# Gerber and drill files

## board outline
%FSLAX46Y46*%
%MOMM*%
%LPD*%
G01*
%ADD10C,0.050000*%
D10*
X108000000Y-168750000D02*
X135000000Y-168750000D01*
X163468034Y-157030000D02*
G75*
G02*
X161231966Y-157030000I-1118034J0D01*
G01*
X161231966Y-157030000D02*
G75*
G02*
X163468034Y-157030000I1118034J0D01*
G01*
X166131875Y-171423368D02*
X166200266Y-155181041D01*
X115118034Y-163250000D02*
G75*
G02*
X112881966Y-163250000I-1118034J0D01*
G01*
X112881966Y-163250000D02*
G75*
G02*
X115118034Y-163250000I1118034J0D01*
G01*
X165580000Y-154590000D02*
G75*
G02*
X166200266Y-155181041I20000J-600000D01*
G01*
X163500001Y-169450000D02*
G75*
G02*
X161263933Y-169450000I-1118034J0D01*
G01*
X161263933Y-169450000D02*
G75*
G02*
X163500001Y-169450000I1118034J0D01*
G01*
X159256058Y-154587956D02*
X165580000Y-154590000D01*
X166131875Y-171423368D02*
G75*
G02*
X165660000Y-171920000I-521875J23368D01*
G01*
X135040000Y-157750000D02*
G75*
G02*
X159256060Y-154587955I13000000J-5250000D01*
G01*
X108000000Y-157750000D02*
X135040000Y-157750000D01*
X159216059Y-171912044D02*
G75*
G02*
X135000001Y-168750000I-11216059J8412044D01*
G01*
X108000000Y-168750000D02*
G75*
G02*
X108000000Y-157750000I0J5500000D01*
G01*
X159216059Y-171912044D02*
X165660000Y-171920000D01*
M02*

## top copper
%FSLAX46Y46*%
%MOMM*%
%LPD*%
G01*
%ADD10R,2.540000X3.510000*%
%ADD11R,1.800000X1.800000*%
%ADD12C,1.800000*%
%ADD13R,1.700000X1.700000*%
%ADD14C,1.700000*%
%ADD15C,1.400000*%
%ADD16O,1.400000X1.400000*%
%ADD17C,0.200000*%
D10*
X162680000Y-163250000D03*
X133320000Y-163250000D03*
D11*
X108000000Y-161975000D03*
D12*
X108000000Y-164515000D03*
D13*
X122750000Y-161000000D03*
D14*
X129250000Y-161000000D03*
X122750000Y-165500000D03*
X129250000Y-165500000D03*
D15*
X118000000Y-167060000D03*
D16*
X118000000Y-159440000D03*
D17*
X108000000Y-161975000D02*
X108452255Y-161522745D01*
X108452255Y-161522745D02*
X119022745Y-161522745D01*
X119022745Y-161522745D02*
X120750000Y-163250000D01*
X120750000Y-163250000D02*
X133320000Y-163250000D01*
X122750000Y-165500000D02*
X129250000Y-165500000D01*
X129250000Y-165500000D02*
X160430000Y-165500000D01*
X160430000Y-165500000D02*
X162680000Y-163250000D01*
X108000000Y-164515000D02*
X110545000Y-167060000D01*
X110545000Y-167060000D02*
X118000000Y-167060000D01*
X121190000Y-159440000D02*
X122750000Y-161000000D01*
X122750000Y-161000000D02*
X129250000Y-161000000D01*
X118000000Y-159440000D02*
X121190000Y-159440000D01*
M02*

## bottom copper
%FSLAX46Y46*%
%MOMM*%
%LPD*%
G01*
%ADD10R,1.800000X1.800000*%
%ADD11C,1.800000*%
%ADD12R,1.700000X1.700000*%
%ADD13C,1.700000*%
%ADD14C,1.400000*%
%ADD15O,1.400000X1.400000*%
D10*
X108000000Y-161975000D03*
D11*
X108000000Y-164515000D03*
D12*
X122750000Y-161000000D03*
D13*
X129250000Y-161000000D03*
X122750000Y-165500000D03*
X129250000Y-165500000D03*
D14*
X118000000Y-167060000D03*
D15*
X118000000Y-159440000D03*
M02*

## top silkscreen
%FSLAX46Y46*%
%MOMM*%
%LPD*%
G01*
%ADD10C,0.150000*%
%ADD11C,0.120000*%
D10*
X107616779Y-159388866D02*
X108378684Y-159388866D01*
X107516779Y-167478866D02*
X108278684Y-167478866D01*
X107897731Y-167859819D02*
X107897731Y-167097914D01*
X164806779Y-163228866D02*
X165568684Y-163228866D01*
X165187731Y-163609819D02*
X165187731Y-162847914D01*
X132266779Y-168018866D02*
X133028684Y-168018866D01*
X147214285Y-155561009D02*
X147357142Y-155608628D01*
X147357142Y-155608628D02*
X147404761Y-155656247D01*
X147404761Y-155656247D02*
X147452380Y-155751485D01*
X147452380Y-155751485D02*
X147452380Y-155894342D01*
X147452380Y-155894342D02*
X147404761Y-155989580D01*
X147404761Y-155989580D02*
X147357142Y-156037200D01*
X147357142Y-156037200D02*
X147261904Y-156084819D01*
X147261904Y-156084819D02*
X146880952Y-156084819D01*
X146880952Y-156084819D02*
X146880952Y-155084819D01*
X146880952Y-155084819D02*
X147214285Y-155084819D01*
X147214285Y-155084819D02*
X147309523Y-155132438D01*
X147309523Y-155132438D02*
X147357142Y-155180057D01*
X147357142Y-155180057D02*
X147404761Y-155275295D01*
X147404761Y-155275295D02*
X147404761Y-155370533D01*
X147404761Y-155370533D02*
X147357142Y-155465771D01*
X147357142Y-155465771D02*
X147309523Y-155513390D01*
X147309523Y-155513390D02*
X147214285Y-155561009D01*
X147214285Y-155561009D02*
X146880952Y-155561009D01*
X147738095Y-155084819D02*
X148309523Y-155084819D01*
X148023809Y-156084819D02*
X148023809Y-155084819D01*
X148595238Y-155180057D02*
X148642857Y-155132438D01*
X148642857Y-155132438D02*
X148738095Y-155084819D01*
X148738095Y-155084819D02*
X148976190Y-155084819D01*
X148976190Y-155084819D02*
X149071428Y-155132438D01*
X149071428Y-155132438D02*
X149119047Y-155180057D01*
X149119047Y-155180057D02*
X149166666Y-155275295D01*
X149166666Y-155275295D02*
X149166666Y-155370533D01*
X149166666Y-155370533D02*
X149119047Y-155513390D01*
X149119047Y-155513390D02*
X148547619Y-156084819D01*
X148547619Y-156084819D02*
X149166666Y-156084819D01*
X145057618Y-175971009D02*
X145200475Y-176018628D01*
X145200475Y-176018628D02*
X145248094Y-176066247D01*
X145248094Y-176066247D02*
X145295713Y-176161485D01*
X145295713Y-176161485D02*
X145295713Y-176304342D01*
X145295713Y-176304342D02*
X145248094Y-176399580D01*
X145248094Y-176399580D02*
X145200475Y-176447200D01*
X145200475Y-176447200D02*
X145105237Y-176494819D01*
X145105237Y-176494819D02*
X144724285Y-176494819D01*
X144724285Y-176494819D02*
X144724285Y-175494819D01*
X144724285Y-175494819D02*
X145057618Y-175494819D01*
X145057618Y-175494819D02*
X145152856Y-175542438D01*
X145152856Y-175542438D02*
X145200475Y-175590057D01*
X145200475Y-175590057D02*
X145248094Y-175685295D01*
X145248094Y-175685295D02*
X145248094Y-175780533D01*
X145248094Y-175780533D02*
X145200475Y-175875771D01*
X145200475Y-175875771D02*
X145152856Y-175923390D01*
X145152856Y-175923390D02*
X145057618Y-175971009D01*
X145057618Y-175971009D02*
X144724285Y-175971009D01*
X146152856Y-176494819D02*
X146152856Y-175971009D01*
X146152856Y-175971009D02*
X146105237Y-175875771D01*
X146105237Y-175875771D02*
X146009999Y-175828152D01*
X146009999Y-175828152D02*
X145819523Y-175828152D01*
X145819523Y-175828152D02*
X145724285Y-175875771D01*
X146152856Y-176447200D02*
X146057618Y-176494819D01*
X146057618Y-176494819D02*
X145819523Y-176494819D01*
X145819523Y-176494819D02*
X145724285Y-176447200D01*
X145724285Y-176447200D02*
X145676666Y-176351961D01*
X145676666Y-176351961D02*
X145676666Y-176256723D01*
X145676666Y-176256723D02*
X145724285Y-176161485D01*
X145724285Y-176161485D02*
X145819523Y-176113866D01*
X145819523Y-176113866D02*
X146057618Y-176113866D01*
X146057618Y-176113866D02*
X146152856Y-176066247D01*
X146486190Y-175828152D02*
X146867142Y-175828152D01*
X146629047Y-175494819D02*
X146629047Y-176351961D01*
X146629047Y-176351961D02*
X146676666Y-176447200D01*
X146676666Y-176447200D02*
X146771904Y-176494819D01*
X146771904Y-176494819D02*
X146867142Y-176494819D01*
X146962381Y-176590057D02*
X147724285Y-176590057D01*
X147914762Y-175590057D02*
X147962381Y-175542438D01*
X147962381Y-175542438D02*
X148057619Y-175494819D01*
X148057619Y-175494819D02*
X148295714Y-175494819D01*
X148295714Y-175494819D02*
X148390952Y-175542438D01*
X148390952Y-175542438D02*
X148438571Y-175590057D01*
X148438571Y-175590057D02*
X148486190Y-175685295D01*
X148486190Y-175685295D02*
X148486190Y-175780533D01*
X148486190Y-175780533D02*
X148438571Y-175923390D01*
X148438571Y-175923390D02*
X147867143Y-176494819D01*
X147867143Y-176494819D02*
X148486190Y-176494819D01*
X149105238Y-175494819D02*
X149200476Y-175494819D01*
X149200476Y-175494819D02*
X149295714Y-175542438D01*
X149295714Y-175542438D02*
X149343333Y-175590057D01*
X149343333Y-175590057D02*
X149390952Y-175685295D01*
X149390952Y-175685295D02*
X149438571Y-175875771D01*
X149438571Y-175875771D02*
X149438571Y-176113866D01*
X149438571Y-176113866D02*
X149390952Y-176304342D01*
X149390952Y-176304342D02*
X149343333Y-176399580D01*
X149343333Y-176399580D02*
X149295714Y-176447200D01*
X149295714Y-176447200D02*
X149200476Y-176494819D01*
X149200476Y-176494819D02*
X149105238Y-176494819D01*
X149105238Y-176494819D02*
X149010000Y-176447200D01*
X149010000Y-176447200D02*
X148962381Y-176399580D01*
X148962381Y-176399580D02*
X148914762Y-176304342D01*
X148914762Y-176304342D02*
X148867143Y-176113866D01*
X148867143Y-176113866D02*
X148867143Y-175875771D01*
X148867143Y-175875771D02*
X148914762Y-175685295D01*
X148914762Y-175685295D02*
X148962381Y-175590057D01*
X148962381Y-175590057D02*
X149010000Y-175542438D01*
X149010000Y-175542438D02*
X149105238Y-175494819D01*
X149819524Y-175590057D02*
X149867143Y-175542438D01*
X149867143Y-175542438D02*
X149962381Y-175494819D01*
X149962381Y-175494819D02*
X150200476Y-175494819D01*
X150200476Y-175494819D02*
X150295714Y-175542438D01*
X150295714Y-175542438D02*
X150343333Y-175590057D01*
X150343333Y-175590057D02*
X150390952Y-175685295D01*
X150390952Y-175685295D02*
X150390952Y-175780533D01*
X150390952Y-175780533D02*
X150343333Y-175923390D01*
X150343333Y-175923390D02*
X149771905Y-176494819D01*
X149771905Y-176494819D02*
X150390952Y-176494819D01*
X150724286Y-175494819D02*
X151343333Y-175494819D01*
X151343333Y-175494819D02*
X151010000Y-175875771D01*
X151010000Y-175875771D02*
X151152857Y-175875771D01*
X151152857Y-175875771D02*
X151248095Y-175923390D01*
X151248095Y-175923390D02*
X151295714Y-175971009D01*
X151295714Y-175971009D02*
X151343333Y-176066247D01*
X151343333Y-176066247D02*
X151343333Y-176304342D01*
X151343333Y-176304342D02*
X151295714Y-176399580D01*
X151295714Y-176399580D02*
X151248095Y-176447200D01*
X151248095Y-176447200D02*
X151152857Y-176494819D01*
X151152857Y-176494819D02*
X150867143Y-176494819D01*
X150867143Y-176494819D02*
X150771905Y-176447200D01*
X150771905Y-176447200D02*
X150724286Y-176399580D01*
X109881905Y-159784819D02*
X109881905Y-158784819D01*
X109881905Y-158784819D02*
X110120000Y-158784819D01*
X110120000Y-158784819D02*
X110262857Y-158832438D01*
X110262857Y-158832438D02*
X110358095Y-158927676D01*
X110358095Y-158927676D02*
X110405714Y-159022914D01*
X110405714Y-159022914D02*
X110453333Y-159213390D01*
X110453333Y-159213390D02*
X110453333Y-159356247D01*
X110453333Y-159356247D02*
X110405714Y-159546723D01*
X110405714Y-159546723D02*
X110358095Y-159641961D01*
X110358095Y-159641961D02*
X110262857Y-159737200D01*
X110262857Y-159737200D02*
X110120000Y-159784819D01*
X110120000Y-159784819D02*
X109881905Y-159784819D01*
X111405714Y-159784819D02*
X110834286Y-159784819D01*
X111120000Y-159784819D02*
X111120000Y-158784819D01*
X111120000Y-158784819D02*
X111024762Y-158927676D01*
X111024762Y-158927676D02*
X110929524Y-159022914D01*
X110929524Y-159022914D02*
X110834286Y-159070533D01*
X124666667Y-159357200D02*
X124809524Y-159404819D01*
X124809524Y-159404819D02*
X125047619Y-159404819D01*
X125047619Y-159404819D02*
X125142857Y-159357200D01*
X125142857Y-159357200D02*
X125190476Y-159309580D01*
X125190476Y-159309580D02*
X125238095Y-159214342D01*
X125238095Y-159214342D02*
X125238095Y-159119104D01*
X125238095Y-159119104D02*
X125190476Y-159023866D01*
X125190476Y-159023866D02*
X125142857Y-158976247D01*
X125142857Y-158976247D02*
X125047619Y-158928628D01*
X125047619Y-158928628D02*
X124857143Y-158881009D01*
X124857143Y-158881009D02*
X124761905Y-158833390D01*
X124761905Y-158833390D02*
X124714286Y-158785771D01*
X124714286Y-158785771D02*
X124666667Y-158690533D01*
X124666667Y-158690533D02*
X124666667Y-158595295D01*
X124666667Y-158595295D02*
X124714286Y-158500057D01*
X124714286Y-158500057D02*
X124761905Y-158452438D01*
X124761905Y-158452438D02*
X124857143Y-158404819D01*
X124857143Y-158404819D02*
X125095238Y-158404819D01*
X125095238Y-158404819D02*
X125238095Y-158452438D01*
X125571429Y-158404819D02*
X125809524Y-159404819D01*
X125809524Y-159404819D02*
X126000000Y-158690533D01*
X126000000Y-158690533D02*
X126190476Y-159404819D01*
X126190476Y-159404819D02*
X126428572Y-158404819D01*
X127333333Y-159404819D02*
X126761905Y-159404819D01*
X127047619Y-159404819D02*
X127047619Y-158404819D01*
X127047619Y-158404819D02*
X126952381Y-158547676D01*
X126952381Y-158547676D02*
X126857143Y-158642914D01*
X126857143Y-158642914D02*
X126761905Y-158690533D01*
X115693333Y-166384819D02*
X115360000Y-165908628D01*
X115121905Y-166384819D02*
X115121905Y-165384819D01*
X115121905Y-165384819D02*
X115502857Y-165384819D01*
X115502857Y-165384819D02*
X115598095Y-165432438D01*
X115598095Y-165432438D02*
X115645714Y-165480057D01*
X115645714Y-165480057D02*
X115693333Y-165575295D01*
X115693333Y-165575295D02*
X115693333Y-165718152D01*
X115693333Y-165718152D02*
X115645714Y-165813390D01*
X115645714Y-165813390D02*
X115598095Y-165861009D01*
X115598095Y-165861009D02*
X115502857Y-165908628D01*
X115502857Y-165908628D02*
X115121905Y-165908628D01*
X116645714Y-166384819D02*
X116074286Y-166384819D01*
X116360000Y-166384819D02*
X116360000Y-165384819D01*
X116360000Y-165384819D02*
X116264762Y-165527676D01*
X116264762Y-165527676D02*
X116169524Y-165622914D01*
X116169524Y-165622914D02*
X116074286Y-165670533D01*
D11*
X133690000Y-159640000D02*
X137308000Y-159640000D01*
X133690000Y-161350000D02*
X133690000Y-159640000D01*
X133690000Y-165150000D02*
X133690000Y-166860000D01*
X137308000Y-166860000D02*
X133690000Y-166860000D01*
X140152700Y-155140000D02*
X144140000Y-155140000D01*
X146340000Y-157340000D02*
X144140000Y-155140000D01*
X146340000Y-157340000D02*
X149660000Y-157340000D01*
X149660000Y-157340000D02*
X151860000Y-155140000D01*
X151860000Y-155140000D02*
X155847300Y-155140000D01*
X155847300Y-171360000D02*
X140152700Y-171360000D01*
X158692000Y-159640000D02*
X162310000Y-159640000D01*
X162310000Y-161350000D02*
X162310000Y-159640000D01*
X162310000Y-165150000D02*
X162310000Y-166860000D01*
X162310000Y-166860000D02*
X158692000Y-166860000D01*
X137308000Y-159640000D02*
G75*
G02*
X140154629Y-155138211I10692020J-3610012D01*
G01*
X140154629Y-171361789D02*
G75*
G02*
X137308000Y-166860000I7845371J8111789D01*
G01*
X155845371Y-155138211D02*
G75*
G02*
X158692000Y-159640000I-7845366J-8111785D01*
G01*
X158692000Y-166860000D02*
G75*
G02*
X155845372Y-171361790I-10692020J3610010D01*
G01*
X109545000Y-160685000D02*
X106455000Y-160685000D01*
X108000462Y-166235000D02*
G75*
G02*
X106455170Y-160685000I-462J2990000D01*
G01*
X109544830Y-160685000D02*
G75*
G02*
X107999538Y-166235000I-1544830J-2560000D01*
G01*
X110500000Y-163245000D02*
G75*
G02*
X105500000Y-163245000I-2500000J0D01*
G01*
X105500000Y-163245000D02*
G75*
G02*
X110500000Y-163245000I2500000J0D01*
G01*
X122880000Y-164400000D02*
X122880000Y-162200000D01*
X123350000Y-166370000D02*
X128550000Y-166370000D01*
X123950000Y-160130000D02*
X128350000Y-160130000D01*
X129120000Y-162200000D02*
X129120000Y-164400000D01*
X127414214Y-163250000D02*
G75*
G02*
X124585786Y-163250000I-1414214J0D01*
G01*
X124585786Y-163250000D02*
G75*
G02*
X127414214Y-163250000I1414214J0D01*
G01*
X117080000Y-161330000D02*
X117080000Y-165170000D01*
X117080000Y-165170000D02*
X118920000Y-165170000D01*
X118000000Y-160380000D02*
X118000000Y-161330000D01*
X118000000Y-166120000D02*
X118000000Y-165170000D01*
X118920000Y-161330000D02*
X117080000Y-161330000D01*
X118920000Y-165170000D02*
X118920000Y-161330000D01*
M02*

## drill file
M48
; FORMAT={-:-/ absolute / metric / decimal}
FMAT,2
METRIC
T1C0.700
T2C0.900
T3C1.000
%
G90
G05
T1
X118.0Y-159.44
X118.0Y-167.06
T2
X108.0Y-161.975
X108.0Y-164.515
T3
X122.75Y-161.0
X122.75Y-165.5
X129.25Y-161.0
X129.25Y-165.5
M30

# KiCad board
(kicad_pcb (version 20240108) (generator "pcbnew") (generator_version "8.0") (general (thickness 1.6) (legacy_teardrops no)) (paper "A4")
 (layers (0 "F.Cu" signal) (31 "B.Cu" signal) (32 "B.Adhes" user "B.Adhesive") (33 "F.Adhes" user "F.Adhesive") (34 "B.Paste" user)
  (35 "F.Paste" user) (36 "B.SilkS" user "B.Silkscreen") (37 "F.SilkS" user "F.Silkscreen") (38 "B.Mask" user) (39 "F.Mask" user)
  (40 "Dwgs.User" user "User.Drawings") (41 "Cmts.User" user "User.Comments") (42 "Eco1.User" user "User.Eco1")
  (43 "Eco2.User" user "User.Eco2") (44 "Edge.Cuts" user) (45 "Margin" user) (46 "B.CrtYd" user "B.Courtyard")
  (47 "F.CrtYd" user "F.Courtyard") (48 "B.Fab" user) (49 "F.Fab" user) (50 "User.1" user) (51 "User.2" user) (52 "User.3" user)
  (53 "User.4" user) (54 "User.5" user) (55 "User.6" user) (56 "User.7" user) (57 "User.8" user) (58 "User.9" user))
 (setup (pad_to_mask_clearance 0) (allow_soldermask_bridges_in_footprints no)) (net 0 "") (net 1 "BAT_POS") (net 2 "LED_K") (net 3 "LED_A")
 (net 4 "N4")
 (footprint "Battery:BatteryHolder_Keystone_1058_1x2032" (layer "F.Cu") (at 148 163.25 180)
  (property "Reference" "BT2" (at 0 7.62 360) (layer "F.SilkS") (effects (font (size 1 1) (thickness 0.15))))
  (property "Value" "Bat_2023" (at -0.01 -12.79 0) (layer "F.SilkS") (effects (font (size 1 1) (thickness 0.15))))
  (fp_line (start 14.31 3.61) (end 10.692 3.61) (stroke (width 0.12) (type solid)) (layer "F.SilkS"))
  (fp_line (start 14.31 1.9) (end 14.31 3.61) (stroke (width 0.12) (type solid)) (layer "F.SilkS"))
  (fp_line (start 14.31 -1.9) (end 14.31 -3.61) (stroke (width 0.12) (type solid)) (layer "F.SilkS"))
  (fp_line (start 10.692 -3.61) (end 14.31 -3.61) (stroke (width 0.12) (type solid)) (layer "F.SilkS"))
  (fp_line (start 7.8473 8.11) (end 3.86 8.11) (stroke (width 0.12) (type solid)) (layer "F.SilkS"))
  (fp_line (start 1.66 5.91) (end 3.86 8.11) (stroke (width 0.12) (type solid)) (layer "F.SilkS"))
  (fp_line (start 1.66 5.91) (end -1.66 5.91) (stroke (width 0.12) (type solid)) (layer "F.SilkS"))
  (fp_line (start -1.66 5.91) (end -3.86 8.11) (stroke (width 0.12) (type solid)) (layer "F.SilkS"))
  (fp_line (start -3.86 8.11) (end -7.8473 8.11) (stroke (width 0.12) (type solid)) (layer "F.SilkS"))
  (fp_line (start -7.8473 -8.11) (end 7.8473 -8.11) (stroke (width 0.12) (type solid)) (layer "F.SilkS"))
  (fp_line (start -10.692 3.61) (end -14.31 3.61) (stroke (width 0.12) (type solid)) (layer "F.SilkS"))
  (fp_line (start -14.31 1.9) (end -14.31 3.61) (stroke (width 0.12) (type solid)) (layer "F.SilkS"))
  (fp_line (start -14.31 -1.9) (end -14.31 -3.61) (stroke (width 0.12) (type solid)) (layer "F.SilkS"))
  (fp_line (start -14.31 -3.61) (end -10.692 -3.61) (stroke (width 0.12) (type solid)) (layer "F.SilkS"))
  (fp_arc (start 10.692 3.61) (mid 9.538084 6.031244) (end 7.845371 8.111789) (stroke (width 0.12) (type solid)) (layer "F.SilkS"))
  (fp_arc (start 7.845371 -8.111789) (mid 9.538085 -6.031244) (end 10.692 -3.61) (stroke (width 0.12) (type solid)) (layer "F.SilkS"))
  (fp_arc (start -7.845371 8.111789) (mid -9.538085 6.031244) (end -10.692 3.61) (stroke (width 0.12) (type solid)) (layer "F.SilkS"))
  (fp_arc (start -10.692 -3.61) (mid -9.538084 -6.031244) (end -7.845371 -8.111789) (stroke (width 0.12) (type solid)) (layer "F.SilkS"))
  (pad "1" smd rect (at -14.68 0 180) (size 2.54 3.51) (layers "F.Cu" "F.Paste" "F.Mask") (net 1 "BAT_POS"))
  (pad "2" smd rect (at 14.68 0 180) (size 2.54 3.51) (layers "F.Cu" "F.Paste" "F.Mask") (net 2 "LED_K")))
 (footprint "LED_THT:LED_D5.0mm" (layer "F.Cu") (at 108 161.975 -90)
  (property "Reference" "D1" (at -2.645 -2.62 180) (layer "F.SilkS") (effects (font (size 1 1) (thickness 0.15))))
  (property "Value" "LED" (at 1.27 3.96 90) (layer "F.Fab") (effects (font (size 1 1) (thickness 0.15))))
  (fp_line (start -1.29 -1.545) (end -1.29 1.545) (stroke (width 0.12) (type solid)) (layer "F.SilkS"))
  (fp_arc (start 4.26 -0.000462) (mid 2.072002 2.880433) (end -1.29 1.54483) (stroke (width 0.12) (type solid)) (layer "F.SilkS"))
  (fp_arc (start -1.29 -1.54483) (mid 2.072002 -2.880433) (end 4.26 0.000462) (stroke (width 0.12) (type solid)) (layer "F.SilkS"))
  (fp_circle (center 1.27 0) (end 3.77 0) (stroke (width 0.12) (type solid)) (fill none) (layer "F.SilkS"))
  (pad "1" thru_hole rect (at 0 0 270) (size 1.8 1.8) (drill 0.9) (layers "*.Cu" "*.Mask") (remove_unused_layers no) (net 2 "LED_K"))
  (pad "2" thru_hole circle (at 2.54 0 270) (size 1.8 1.8) (drill 0.9) (layers "*.Cu" "*.Mask") (remove_unused_layers no) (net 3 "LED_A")))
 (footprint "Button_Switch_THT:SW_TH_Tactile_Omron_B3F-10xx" (layer "F.Cu") (at 122.75 161)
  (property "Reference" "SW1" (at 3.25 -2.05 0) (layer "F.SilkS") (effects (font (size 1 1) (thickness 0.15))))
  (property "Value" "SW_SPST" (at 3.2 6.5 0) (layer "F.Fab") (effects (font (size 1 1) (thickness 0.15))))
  (fp_line (start 0.13 3.4) (end 0.13 1.2) (stroke (width 0.12) (type solid)) (layer "F.SilkS"))
  (fp_line (start 0.6 5.37) (end 5.8 5.37) (stroke (width 0.12) (type solid)) (layer "F.SilkS"))
  (fp_line (start 1.2 -0.87) (end 5.6 -0.87) (stroke (width 0.12) (type solid)) (layer "F.SilkS"))
  (fp_line (start 6.37 1.2) (end 6.37 3.4) (stroke (width 0.12) (type solid)) (layer "F.SilkS"))
  (fp_circle (center 3.25 2.25) (end 4.25 3.25) (stroke (width 0.12) (type solid)) (fill none) (layer "F.SilkS"))
  (pad "1" thru_hole rect (at 0 0) (size 1.7 1.7) (drill 1) (layers "*.Cu" "*.Mask") (remove_unused_layers no) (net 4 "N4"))
  (pad "1" thru_hole circle (at 6.5 0) (size 1.7 1.7) (drill 1) (layers "*.Cu" "*.Mask") (remove_unused_layers no) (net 4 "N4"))
  (pad "2" thru_hole circle (at 0 4.5) (size 1.7 1.7) (drill 1) (layers "*.Cu" "*.Mask") (remove_unused_layers no) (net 1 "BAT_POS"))
  (pad "2" thru_hole circle (at 6.5 4.5) (size 1.7 1.7) (drill 1) (layers "*.Cu" "*.Mask") (remove_unused_layers no) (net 1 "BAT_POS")))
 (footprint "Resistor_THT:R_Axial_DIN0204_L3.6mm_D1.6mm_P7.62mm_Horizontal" (layer "F.Cu") (at 118 167.06 90)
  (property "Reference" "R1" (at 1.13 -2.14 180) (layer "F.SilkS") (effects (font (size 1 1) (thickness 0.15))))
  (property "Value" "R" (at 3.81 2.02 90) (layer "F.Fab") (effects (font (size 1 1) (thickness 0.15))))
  (fp_line (start 5.73 -0.92) (end 1.89 -0.92) (stroke (width 0.12) (type solid)) (layer "F.SilkS"))
  (fp_line (start 1.89 -0.92) (end 1.89 0.92) (stroke (width 0.12) (type solid)) (layer "F.SilkS"))
  (fp_line (start 6.68 0) (end 5.73 0) (stroke (width 0.12) (type solid)) (layer "F.SilkS"))
  (fp_line (start 0.94 0) (end 1.89 0) (stroke (width 0.12) (type solid)) (layer "F.SilkS"))
  (fp_line (start 5.73 0.92) (end 5.73 -0.92) (stroke (width 0.12) (type solid)) (layer "F.SilkS"))
  (fp_line (start 1.89 0.92) (end 5.73 0.92) (stroke (width 0.12) (type solid)) (layer "F.SilkS"))
  (pad "1" thru_hole circle (at 0 0 90) (size 1.4 1.4) (drill 0.7) (layers "*.Cu" "*.Mask") (remove_unused_layers no) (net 3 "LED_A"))
  (pad "2" thru_hole oval (at 7.62 0 90) (size 1.4 1.4) (drill 0.7) (layers "*.Cu" "*.Mask") (remove_unused_layers no) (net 4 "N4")))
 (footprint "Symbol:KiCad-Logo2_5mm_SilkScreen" (layer "B.Cu") (at 148.02 163.44 180)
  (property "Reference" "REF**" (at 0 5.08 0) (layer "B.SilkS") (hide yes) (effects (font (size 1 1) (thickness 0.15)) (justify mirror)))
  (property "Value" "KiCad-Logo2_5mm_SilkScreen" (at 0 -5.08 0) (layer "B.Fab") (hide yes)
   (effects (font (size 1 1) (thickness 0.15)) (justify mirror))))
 (gr_line (start 108 168.75) (end 135 168.75) (locked yes) (stroke (width 0.05) (type default)) (layer "Edge.Cuts"))
 (gr_circle (center 162.35 157.03) (end 163.35 157.53) (locked yes) (stroke (width 0.05) (type default)) (fill none) (layer "Edge.Cuts"))
 (gr_line (start 166.131875 171.423368) (end 166.200266 155.181041) (locked yes) (stroke (width 0.05) (type default)) (layer "Edge.Cuts"))
 (gr_circle (center 114 163.25) (end 115 163.75) (locked yes) (stroke (width 0.05) (type default)) (fill none) (layer "Edge.Cuts"))
 (gr_arc (start 165.58 154.59) (mid 166.014137 154.755385) (end 166.200266 155.181041) (locked yes) (stroke (width 0.05) (type default))
  (layer "Edge.Cuts"))
 (gr_circle (center 162.381967 169.45) (end 163.381967 169.95) (locked yes) (stroke (width 0.05) (type default)) (fill none)
  (layer "Edge.Cuts"))
 (gr_line (start 159.256058 154.587956) (end 165.58 154.59) (locked yes) (stroke (width 0.05) (type default)) (layer "Edge.Cuts"))
 (gr_arc (start 166.131875 171.423368) (mid 165.98871 171.759831) (end 165.66 171.92) (locked yes) (stroke (width 0.05) (type default))
  (layer "Edge.Cuts"))
 (gr_arc (start 135.04 157.75) (mid 146.224719 149.097942) (end 159.256058 154.587956) (locked yes) (stroke (width 0.05) (type default))
  (layer "Edge.Cuts"))
 (gr_line (start 108 157.75) (end 135.04 157.75) (locked yes) (stroke (width 0.05) (type default)) (layer "Edge.Cuts"))
 (gr_arc (start 159.216059 171.912044) (mid 146.18472 177.402058) (end 135.000001 168.75) (locked yes) (stroke (width 0.05) (type default))
  (layer "Edge.Cuts"))
 (gr_arc (start 108 168.75) (mid 102.5 163.25) (end 108 157.75) (locked yes) (stroke (width 0.05) (type default)) (layer "Edge.Cuts"))
 (gr_line (start 159.216059 171.912044) (end 165.66 171.92) (locked yes) (stroke (width 0.05) (type default)) (layer "Edge.Cuts"))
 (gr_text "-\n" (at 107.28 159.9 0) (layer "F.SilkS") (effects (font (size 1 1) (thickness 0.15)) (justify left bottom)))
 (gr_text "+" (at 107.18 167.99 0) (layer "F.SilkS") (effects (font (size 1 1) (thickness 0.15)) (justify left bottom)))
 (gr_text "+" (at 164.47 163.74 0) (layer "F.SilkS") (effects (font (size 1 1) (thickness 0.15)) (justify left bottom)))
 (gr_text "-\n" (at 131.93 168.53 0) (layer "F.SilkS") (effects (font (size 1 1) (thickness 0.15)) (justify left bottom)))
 (segment (start 108 161.975) (end 108.452255 161.522745) (width 0.2) (layer "F.Cu") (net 2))
 (segment (start 108.452255 161.522745) (end 119.022745 161.522745) (width 0.2) (layer "F.Cu") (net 2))
 (segment (start 119.022745 161.522745) (end 120.75 163.25) (width 0.2) (layer "F.Cu") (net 2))
 (segment (start 120.75 163.25) (end 133.32 163.25) (width 0.2) (layer "F.Cu") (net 2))
 (segment (start 122.75 165.5) (end 129.25 165.5) (width 0.2) (layer "F.Cu") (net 1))
 (segment (start 129.25 165.5) (end 160.43 165.5) (width 0.2) (layer "F.Cu") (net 1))
 (segment (start 160.43 165.5) (end 162.68 163.25) (width 0.2) (layer "F.Cu") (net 1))
 (segment (start 108 164.515) (end 110.545 167.06) (width 0.2) (layer "F.Cu") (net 3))
 (segment (start 110.545 167.06) (end 118 167.06) (width 0.2) (layer "F.Cu") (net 3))
 (segment (start 121.19 159.44) (end 122.75 161) (width 0.2) (layer "F.Cu") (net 4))
 (segment (start 122.75 161) (end 129.25 161) (width 0.2) (layer "F.Cu") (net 4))
 (segment (start 118 159.44) (end 121.19 159.44) (width 0.2) (layer "F.Cu") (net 4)))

